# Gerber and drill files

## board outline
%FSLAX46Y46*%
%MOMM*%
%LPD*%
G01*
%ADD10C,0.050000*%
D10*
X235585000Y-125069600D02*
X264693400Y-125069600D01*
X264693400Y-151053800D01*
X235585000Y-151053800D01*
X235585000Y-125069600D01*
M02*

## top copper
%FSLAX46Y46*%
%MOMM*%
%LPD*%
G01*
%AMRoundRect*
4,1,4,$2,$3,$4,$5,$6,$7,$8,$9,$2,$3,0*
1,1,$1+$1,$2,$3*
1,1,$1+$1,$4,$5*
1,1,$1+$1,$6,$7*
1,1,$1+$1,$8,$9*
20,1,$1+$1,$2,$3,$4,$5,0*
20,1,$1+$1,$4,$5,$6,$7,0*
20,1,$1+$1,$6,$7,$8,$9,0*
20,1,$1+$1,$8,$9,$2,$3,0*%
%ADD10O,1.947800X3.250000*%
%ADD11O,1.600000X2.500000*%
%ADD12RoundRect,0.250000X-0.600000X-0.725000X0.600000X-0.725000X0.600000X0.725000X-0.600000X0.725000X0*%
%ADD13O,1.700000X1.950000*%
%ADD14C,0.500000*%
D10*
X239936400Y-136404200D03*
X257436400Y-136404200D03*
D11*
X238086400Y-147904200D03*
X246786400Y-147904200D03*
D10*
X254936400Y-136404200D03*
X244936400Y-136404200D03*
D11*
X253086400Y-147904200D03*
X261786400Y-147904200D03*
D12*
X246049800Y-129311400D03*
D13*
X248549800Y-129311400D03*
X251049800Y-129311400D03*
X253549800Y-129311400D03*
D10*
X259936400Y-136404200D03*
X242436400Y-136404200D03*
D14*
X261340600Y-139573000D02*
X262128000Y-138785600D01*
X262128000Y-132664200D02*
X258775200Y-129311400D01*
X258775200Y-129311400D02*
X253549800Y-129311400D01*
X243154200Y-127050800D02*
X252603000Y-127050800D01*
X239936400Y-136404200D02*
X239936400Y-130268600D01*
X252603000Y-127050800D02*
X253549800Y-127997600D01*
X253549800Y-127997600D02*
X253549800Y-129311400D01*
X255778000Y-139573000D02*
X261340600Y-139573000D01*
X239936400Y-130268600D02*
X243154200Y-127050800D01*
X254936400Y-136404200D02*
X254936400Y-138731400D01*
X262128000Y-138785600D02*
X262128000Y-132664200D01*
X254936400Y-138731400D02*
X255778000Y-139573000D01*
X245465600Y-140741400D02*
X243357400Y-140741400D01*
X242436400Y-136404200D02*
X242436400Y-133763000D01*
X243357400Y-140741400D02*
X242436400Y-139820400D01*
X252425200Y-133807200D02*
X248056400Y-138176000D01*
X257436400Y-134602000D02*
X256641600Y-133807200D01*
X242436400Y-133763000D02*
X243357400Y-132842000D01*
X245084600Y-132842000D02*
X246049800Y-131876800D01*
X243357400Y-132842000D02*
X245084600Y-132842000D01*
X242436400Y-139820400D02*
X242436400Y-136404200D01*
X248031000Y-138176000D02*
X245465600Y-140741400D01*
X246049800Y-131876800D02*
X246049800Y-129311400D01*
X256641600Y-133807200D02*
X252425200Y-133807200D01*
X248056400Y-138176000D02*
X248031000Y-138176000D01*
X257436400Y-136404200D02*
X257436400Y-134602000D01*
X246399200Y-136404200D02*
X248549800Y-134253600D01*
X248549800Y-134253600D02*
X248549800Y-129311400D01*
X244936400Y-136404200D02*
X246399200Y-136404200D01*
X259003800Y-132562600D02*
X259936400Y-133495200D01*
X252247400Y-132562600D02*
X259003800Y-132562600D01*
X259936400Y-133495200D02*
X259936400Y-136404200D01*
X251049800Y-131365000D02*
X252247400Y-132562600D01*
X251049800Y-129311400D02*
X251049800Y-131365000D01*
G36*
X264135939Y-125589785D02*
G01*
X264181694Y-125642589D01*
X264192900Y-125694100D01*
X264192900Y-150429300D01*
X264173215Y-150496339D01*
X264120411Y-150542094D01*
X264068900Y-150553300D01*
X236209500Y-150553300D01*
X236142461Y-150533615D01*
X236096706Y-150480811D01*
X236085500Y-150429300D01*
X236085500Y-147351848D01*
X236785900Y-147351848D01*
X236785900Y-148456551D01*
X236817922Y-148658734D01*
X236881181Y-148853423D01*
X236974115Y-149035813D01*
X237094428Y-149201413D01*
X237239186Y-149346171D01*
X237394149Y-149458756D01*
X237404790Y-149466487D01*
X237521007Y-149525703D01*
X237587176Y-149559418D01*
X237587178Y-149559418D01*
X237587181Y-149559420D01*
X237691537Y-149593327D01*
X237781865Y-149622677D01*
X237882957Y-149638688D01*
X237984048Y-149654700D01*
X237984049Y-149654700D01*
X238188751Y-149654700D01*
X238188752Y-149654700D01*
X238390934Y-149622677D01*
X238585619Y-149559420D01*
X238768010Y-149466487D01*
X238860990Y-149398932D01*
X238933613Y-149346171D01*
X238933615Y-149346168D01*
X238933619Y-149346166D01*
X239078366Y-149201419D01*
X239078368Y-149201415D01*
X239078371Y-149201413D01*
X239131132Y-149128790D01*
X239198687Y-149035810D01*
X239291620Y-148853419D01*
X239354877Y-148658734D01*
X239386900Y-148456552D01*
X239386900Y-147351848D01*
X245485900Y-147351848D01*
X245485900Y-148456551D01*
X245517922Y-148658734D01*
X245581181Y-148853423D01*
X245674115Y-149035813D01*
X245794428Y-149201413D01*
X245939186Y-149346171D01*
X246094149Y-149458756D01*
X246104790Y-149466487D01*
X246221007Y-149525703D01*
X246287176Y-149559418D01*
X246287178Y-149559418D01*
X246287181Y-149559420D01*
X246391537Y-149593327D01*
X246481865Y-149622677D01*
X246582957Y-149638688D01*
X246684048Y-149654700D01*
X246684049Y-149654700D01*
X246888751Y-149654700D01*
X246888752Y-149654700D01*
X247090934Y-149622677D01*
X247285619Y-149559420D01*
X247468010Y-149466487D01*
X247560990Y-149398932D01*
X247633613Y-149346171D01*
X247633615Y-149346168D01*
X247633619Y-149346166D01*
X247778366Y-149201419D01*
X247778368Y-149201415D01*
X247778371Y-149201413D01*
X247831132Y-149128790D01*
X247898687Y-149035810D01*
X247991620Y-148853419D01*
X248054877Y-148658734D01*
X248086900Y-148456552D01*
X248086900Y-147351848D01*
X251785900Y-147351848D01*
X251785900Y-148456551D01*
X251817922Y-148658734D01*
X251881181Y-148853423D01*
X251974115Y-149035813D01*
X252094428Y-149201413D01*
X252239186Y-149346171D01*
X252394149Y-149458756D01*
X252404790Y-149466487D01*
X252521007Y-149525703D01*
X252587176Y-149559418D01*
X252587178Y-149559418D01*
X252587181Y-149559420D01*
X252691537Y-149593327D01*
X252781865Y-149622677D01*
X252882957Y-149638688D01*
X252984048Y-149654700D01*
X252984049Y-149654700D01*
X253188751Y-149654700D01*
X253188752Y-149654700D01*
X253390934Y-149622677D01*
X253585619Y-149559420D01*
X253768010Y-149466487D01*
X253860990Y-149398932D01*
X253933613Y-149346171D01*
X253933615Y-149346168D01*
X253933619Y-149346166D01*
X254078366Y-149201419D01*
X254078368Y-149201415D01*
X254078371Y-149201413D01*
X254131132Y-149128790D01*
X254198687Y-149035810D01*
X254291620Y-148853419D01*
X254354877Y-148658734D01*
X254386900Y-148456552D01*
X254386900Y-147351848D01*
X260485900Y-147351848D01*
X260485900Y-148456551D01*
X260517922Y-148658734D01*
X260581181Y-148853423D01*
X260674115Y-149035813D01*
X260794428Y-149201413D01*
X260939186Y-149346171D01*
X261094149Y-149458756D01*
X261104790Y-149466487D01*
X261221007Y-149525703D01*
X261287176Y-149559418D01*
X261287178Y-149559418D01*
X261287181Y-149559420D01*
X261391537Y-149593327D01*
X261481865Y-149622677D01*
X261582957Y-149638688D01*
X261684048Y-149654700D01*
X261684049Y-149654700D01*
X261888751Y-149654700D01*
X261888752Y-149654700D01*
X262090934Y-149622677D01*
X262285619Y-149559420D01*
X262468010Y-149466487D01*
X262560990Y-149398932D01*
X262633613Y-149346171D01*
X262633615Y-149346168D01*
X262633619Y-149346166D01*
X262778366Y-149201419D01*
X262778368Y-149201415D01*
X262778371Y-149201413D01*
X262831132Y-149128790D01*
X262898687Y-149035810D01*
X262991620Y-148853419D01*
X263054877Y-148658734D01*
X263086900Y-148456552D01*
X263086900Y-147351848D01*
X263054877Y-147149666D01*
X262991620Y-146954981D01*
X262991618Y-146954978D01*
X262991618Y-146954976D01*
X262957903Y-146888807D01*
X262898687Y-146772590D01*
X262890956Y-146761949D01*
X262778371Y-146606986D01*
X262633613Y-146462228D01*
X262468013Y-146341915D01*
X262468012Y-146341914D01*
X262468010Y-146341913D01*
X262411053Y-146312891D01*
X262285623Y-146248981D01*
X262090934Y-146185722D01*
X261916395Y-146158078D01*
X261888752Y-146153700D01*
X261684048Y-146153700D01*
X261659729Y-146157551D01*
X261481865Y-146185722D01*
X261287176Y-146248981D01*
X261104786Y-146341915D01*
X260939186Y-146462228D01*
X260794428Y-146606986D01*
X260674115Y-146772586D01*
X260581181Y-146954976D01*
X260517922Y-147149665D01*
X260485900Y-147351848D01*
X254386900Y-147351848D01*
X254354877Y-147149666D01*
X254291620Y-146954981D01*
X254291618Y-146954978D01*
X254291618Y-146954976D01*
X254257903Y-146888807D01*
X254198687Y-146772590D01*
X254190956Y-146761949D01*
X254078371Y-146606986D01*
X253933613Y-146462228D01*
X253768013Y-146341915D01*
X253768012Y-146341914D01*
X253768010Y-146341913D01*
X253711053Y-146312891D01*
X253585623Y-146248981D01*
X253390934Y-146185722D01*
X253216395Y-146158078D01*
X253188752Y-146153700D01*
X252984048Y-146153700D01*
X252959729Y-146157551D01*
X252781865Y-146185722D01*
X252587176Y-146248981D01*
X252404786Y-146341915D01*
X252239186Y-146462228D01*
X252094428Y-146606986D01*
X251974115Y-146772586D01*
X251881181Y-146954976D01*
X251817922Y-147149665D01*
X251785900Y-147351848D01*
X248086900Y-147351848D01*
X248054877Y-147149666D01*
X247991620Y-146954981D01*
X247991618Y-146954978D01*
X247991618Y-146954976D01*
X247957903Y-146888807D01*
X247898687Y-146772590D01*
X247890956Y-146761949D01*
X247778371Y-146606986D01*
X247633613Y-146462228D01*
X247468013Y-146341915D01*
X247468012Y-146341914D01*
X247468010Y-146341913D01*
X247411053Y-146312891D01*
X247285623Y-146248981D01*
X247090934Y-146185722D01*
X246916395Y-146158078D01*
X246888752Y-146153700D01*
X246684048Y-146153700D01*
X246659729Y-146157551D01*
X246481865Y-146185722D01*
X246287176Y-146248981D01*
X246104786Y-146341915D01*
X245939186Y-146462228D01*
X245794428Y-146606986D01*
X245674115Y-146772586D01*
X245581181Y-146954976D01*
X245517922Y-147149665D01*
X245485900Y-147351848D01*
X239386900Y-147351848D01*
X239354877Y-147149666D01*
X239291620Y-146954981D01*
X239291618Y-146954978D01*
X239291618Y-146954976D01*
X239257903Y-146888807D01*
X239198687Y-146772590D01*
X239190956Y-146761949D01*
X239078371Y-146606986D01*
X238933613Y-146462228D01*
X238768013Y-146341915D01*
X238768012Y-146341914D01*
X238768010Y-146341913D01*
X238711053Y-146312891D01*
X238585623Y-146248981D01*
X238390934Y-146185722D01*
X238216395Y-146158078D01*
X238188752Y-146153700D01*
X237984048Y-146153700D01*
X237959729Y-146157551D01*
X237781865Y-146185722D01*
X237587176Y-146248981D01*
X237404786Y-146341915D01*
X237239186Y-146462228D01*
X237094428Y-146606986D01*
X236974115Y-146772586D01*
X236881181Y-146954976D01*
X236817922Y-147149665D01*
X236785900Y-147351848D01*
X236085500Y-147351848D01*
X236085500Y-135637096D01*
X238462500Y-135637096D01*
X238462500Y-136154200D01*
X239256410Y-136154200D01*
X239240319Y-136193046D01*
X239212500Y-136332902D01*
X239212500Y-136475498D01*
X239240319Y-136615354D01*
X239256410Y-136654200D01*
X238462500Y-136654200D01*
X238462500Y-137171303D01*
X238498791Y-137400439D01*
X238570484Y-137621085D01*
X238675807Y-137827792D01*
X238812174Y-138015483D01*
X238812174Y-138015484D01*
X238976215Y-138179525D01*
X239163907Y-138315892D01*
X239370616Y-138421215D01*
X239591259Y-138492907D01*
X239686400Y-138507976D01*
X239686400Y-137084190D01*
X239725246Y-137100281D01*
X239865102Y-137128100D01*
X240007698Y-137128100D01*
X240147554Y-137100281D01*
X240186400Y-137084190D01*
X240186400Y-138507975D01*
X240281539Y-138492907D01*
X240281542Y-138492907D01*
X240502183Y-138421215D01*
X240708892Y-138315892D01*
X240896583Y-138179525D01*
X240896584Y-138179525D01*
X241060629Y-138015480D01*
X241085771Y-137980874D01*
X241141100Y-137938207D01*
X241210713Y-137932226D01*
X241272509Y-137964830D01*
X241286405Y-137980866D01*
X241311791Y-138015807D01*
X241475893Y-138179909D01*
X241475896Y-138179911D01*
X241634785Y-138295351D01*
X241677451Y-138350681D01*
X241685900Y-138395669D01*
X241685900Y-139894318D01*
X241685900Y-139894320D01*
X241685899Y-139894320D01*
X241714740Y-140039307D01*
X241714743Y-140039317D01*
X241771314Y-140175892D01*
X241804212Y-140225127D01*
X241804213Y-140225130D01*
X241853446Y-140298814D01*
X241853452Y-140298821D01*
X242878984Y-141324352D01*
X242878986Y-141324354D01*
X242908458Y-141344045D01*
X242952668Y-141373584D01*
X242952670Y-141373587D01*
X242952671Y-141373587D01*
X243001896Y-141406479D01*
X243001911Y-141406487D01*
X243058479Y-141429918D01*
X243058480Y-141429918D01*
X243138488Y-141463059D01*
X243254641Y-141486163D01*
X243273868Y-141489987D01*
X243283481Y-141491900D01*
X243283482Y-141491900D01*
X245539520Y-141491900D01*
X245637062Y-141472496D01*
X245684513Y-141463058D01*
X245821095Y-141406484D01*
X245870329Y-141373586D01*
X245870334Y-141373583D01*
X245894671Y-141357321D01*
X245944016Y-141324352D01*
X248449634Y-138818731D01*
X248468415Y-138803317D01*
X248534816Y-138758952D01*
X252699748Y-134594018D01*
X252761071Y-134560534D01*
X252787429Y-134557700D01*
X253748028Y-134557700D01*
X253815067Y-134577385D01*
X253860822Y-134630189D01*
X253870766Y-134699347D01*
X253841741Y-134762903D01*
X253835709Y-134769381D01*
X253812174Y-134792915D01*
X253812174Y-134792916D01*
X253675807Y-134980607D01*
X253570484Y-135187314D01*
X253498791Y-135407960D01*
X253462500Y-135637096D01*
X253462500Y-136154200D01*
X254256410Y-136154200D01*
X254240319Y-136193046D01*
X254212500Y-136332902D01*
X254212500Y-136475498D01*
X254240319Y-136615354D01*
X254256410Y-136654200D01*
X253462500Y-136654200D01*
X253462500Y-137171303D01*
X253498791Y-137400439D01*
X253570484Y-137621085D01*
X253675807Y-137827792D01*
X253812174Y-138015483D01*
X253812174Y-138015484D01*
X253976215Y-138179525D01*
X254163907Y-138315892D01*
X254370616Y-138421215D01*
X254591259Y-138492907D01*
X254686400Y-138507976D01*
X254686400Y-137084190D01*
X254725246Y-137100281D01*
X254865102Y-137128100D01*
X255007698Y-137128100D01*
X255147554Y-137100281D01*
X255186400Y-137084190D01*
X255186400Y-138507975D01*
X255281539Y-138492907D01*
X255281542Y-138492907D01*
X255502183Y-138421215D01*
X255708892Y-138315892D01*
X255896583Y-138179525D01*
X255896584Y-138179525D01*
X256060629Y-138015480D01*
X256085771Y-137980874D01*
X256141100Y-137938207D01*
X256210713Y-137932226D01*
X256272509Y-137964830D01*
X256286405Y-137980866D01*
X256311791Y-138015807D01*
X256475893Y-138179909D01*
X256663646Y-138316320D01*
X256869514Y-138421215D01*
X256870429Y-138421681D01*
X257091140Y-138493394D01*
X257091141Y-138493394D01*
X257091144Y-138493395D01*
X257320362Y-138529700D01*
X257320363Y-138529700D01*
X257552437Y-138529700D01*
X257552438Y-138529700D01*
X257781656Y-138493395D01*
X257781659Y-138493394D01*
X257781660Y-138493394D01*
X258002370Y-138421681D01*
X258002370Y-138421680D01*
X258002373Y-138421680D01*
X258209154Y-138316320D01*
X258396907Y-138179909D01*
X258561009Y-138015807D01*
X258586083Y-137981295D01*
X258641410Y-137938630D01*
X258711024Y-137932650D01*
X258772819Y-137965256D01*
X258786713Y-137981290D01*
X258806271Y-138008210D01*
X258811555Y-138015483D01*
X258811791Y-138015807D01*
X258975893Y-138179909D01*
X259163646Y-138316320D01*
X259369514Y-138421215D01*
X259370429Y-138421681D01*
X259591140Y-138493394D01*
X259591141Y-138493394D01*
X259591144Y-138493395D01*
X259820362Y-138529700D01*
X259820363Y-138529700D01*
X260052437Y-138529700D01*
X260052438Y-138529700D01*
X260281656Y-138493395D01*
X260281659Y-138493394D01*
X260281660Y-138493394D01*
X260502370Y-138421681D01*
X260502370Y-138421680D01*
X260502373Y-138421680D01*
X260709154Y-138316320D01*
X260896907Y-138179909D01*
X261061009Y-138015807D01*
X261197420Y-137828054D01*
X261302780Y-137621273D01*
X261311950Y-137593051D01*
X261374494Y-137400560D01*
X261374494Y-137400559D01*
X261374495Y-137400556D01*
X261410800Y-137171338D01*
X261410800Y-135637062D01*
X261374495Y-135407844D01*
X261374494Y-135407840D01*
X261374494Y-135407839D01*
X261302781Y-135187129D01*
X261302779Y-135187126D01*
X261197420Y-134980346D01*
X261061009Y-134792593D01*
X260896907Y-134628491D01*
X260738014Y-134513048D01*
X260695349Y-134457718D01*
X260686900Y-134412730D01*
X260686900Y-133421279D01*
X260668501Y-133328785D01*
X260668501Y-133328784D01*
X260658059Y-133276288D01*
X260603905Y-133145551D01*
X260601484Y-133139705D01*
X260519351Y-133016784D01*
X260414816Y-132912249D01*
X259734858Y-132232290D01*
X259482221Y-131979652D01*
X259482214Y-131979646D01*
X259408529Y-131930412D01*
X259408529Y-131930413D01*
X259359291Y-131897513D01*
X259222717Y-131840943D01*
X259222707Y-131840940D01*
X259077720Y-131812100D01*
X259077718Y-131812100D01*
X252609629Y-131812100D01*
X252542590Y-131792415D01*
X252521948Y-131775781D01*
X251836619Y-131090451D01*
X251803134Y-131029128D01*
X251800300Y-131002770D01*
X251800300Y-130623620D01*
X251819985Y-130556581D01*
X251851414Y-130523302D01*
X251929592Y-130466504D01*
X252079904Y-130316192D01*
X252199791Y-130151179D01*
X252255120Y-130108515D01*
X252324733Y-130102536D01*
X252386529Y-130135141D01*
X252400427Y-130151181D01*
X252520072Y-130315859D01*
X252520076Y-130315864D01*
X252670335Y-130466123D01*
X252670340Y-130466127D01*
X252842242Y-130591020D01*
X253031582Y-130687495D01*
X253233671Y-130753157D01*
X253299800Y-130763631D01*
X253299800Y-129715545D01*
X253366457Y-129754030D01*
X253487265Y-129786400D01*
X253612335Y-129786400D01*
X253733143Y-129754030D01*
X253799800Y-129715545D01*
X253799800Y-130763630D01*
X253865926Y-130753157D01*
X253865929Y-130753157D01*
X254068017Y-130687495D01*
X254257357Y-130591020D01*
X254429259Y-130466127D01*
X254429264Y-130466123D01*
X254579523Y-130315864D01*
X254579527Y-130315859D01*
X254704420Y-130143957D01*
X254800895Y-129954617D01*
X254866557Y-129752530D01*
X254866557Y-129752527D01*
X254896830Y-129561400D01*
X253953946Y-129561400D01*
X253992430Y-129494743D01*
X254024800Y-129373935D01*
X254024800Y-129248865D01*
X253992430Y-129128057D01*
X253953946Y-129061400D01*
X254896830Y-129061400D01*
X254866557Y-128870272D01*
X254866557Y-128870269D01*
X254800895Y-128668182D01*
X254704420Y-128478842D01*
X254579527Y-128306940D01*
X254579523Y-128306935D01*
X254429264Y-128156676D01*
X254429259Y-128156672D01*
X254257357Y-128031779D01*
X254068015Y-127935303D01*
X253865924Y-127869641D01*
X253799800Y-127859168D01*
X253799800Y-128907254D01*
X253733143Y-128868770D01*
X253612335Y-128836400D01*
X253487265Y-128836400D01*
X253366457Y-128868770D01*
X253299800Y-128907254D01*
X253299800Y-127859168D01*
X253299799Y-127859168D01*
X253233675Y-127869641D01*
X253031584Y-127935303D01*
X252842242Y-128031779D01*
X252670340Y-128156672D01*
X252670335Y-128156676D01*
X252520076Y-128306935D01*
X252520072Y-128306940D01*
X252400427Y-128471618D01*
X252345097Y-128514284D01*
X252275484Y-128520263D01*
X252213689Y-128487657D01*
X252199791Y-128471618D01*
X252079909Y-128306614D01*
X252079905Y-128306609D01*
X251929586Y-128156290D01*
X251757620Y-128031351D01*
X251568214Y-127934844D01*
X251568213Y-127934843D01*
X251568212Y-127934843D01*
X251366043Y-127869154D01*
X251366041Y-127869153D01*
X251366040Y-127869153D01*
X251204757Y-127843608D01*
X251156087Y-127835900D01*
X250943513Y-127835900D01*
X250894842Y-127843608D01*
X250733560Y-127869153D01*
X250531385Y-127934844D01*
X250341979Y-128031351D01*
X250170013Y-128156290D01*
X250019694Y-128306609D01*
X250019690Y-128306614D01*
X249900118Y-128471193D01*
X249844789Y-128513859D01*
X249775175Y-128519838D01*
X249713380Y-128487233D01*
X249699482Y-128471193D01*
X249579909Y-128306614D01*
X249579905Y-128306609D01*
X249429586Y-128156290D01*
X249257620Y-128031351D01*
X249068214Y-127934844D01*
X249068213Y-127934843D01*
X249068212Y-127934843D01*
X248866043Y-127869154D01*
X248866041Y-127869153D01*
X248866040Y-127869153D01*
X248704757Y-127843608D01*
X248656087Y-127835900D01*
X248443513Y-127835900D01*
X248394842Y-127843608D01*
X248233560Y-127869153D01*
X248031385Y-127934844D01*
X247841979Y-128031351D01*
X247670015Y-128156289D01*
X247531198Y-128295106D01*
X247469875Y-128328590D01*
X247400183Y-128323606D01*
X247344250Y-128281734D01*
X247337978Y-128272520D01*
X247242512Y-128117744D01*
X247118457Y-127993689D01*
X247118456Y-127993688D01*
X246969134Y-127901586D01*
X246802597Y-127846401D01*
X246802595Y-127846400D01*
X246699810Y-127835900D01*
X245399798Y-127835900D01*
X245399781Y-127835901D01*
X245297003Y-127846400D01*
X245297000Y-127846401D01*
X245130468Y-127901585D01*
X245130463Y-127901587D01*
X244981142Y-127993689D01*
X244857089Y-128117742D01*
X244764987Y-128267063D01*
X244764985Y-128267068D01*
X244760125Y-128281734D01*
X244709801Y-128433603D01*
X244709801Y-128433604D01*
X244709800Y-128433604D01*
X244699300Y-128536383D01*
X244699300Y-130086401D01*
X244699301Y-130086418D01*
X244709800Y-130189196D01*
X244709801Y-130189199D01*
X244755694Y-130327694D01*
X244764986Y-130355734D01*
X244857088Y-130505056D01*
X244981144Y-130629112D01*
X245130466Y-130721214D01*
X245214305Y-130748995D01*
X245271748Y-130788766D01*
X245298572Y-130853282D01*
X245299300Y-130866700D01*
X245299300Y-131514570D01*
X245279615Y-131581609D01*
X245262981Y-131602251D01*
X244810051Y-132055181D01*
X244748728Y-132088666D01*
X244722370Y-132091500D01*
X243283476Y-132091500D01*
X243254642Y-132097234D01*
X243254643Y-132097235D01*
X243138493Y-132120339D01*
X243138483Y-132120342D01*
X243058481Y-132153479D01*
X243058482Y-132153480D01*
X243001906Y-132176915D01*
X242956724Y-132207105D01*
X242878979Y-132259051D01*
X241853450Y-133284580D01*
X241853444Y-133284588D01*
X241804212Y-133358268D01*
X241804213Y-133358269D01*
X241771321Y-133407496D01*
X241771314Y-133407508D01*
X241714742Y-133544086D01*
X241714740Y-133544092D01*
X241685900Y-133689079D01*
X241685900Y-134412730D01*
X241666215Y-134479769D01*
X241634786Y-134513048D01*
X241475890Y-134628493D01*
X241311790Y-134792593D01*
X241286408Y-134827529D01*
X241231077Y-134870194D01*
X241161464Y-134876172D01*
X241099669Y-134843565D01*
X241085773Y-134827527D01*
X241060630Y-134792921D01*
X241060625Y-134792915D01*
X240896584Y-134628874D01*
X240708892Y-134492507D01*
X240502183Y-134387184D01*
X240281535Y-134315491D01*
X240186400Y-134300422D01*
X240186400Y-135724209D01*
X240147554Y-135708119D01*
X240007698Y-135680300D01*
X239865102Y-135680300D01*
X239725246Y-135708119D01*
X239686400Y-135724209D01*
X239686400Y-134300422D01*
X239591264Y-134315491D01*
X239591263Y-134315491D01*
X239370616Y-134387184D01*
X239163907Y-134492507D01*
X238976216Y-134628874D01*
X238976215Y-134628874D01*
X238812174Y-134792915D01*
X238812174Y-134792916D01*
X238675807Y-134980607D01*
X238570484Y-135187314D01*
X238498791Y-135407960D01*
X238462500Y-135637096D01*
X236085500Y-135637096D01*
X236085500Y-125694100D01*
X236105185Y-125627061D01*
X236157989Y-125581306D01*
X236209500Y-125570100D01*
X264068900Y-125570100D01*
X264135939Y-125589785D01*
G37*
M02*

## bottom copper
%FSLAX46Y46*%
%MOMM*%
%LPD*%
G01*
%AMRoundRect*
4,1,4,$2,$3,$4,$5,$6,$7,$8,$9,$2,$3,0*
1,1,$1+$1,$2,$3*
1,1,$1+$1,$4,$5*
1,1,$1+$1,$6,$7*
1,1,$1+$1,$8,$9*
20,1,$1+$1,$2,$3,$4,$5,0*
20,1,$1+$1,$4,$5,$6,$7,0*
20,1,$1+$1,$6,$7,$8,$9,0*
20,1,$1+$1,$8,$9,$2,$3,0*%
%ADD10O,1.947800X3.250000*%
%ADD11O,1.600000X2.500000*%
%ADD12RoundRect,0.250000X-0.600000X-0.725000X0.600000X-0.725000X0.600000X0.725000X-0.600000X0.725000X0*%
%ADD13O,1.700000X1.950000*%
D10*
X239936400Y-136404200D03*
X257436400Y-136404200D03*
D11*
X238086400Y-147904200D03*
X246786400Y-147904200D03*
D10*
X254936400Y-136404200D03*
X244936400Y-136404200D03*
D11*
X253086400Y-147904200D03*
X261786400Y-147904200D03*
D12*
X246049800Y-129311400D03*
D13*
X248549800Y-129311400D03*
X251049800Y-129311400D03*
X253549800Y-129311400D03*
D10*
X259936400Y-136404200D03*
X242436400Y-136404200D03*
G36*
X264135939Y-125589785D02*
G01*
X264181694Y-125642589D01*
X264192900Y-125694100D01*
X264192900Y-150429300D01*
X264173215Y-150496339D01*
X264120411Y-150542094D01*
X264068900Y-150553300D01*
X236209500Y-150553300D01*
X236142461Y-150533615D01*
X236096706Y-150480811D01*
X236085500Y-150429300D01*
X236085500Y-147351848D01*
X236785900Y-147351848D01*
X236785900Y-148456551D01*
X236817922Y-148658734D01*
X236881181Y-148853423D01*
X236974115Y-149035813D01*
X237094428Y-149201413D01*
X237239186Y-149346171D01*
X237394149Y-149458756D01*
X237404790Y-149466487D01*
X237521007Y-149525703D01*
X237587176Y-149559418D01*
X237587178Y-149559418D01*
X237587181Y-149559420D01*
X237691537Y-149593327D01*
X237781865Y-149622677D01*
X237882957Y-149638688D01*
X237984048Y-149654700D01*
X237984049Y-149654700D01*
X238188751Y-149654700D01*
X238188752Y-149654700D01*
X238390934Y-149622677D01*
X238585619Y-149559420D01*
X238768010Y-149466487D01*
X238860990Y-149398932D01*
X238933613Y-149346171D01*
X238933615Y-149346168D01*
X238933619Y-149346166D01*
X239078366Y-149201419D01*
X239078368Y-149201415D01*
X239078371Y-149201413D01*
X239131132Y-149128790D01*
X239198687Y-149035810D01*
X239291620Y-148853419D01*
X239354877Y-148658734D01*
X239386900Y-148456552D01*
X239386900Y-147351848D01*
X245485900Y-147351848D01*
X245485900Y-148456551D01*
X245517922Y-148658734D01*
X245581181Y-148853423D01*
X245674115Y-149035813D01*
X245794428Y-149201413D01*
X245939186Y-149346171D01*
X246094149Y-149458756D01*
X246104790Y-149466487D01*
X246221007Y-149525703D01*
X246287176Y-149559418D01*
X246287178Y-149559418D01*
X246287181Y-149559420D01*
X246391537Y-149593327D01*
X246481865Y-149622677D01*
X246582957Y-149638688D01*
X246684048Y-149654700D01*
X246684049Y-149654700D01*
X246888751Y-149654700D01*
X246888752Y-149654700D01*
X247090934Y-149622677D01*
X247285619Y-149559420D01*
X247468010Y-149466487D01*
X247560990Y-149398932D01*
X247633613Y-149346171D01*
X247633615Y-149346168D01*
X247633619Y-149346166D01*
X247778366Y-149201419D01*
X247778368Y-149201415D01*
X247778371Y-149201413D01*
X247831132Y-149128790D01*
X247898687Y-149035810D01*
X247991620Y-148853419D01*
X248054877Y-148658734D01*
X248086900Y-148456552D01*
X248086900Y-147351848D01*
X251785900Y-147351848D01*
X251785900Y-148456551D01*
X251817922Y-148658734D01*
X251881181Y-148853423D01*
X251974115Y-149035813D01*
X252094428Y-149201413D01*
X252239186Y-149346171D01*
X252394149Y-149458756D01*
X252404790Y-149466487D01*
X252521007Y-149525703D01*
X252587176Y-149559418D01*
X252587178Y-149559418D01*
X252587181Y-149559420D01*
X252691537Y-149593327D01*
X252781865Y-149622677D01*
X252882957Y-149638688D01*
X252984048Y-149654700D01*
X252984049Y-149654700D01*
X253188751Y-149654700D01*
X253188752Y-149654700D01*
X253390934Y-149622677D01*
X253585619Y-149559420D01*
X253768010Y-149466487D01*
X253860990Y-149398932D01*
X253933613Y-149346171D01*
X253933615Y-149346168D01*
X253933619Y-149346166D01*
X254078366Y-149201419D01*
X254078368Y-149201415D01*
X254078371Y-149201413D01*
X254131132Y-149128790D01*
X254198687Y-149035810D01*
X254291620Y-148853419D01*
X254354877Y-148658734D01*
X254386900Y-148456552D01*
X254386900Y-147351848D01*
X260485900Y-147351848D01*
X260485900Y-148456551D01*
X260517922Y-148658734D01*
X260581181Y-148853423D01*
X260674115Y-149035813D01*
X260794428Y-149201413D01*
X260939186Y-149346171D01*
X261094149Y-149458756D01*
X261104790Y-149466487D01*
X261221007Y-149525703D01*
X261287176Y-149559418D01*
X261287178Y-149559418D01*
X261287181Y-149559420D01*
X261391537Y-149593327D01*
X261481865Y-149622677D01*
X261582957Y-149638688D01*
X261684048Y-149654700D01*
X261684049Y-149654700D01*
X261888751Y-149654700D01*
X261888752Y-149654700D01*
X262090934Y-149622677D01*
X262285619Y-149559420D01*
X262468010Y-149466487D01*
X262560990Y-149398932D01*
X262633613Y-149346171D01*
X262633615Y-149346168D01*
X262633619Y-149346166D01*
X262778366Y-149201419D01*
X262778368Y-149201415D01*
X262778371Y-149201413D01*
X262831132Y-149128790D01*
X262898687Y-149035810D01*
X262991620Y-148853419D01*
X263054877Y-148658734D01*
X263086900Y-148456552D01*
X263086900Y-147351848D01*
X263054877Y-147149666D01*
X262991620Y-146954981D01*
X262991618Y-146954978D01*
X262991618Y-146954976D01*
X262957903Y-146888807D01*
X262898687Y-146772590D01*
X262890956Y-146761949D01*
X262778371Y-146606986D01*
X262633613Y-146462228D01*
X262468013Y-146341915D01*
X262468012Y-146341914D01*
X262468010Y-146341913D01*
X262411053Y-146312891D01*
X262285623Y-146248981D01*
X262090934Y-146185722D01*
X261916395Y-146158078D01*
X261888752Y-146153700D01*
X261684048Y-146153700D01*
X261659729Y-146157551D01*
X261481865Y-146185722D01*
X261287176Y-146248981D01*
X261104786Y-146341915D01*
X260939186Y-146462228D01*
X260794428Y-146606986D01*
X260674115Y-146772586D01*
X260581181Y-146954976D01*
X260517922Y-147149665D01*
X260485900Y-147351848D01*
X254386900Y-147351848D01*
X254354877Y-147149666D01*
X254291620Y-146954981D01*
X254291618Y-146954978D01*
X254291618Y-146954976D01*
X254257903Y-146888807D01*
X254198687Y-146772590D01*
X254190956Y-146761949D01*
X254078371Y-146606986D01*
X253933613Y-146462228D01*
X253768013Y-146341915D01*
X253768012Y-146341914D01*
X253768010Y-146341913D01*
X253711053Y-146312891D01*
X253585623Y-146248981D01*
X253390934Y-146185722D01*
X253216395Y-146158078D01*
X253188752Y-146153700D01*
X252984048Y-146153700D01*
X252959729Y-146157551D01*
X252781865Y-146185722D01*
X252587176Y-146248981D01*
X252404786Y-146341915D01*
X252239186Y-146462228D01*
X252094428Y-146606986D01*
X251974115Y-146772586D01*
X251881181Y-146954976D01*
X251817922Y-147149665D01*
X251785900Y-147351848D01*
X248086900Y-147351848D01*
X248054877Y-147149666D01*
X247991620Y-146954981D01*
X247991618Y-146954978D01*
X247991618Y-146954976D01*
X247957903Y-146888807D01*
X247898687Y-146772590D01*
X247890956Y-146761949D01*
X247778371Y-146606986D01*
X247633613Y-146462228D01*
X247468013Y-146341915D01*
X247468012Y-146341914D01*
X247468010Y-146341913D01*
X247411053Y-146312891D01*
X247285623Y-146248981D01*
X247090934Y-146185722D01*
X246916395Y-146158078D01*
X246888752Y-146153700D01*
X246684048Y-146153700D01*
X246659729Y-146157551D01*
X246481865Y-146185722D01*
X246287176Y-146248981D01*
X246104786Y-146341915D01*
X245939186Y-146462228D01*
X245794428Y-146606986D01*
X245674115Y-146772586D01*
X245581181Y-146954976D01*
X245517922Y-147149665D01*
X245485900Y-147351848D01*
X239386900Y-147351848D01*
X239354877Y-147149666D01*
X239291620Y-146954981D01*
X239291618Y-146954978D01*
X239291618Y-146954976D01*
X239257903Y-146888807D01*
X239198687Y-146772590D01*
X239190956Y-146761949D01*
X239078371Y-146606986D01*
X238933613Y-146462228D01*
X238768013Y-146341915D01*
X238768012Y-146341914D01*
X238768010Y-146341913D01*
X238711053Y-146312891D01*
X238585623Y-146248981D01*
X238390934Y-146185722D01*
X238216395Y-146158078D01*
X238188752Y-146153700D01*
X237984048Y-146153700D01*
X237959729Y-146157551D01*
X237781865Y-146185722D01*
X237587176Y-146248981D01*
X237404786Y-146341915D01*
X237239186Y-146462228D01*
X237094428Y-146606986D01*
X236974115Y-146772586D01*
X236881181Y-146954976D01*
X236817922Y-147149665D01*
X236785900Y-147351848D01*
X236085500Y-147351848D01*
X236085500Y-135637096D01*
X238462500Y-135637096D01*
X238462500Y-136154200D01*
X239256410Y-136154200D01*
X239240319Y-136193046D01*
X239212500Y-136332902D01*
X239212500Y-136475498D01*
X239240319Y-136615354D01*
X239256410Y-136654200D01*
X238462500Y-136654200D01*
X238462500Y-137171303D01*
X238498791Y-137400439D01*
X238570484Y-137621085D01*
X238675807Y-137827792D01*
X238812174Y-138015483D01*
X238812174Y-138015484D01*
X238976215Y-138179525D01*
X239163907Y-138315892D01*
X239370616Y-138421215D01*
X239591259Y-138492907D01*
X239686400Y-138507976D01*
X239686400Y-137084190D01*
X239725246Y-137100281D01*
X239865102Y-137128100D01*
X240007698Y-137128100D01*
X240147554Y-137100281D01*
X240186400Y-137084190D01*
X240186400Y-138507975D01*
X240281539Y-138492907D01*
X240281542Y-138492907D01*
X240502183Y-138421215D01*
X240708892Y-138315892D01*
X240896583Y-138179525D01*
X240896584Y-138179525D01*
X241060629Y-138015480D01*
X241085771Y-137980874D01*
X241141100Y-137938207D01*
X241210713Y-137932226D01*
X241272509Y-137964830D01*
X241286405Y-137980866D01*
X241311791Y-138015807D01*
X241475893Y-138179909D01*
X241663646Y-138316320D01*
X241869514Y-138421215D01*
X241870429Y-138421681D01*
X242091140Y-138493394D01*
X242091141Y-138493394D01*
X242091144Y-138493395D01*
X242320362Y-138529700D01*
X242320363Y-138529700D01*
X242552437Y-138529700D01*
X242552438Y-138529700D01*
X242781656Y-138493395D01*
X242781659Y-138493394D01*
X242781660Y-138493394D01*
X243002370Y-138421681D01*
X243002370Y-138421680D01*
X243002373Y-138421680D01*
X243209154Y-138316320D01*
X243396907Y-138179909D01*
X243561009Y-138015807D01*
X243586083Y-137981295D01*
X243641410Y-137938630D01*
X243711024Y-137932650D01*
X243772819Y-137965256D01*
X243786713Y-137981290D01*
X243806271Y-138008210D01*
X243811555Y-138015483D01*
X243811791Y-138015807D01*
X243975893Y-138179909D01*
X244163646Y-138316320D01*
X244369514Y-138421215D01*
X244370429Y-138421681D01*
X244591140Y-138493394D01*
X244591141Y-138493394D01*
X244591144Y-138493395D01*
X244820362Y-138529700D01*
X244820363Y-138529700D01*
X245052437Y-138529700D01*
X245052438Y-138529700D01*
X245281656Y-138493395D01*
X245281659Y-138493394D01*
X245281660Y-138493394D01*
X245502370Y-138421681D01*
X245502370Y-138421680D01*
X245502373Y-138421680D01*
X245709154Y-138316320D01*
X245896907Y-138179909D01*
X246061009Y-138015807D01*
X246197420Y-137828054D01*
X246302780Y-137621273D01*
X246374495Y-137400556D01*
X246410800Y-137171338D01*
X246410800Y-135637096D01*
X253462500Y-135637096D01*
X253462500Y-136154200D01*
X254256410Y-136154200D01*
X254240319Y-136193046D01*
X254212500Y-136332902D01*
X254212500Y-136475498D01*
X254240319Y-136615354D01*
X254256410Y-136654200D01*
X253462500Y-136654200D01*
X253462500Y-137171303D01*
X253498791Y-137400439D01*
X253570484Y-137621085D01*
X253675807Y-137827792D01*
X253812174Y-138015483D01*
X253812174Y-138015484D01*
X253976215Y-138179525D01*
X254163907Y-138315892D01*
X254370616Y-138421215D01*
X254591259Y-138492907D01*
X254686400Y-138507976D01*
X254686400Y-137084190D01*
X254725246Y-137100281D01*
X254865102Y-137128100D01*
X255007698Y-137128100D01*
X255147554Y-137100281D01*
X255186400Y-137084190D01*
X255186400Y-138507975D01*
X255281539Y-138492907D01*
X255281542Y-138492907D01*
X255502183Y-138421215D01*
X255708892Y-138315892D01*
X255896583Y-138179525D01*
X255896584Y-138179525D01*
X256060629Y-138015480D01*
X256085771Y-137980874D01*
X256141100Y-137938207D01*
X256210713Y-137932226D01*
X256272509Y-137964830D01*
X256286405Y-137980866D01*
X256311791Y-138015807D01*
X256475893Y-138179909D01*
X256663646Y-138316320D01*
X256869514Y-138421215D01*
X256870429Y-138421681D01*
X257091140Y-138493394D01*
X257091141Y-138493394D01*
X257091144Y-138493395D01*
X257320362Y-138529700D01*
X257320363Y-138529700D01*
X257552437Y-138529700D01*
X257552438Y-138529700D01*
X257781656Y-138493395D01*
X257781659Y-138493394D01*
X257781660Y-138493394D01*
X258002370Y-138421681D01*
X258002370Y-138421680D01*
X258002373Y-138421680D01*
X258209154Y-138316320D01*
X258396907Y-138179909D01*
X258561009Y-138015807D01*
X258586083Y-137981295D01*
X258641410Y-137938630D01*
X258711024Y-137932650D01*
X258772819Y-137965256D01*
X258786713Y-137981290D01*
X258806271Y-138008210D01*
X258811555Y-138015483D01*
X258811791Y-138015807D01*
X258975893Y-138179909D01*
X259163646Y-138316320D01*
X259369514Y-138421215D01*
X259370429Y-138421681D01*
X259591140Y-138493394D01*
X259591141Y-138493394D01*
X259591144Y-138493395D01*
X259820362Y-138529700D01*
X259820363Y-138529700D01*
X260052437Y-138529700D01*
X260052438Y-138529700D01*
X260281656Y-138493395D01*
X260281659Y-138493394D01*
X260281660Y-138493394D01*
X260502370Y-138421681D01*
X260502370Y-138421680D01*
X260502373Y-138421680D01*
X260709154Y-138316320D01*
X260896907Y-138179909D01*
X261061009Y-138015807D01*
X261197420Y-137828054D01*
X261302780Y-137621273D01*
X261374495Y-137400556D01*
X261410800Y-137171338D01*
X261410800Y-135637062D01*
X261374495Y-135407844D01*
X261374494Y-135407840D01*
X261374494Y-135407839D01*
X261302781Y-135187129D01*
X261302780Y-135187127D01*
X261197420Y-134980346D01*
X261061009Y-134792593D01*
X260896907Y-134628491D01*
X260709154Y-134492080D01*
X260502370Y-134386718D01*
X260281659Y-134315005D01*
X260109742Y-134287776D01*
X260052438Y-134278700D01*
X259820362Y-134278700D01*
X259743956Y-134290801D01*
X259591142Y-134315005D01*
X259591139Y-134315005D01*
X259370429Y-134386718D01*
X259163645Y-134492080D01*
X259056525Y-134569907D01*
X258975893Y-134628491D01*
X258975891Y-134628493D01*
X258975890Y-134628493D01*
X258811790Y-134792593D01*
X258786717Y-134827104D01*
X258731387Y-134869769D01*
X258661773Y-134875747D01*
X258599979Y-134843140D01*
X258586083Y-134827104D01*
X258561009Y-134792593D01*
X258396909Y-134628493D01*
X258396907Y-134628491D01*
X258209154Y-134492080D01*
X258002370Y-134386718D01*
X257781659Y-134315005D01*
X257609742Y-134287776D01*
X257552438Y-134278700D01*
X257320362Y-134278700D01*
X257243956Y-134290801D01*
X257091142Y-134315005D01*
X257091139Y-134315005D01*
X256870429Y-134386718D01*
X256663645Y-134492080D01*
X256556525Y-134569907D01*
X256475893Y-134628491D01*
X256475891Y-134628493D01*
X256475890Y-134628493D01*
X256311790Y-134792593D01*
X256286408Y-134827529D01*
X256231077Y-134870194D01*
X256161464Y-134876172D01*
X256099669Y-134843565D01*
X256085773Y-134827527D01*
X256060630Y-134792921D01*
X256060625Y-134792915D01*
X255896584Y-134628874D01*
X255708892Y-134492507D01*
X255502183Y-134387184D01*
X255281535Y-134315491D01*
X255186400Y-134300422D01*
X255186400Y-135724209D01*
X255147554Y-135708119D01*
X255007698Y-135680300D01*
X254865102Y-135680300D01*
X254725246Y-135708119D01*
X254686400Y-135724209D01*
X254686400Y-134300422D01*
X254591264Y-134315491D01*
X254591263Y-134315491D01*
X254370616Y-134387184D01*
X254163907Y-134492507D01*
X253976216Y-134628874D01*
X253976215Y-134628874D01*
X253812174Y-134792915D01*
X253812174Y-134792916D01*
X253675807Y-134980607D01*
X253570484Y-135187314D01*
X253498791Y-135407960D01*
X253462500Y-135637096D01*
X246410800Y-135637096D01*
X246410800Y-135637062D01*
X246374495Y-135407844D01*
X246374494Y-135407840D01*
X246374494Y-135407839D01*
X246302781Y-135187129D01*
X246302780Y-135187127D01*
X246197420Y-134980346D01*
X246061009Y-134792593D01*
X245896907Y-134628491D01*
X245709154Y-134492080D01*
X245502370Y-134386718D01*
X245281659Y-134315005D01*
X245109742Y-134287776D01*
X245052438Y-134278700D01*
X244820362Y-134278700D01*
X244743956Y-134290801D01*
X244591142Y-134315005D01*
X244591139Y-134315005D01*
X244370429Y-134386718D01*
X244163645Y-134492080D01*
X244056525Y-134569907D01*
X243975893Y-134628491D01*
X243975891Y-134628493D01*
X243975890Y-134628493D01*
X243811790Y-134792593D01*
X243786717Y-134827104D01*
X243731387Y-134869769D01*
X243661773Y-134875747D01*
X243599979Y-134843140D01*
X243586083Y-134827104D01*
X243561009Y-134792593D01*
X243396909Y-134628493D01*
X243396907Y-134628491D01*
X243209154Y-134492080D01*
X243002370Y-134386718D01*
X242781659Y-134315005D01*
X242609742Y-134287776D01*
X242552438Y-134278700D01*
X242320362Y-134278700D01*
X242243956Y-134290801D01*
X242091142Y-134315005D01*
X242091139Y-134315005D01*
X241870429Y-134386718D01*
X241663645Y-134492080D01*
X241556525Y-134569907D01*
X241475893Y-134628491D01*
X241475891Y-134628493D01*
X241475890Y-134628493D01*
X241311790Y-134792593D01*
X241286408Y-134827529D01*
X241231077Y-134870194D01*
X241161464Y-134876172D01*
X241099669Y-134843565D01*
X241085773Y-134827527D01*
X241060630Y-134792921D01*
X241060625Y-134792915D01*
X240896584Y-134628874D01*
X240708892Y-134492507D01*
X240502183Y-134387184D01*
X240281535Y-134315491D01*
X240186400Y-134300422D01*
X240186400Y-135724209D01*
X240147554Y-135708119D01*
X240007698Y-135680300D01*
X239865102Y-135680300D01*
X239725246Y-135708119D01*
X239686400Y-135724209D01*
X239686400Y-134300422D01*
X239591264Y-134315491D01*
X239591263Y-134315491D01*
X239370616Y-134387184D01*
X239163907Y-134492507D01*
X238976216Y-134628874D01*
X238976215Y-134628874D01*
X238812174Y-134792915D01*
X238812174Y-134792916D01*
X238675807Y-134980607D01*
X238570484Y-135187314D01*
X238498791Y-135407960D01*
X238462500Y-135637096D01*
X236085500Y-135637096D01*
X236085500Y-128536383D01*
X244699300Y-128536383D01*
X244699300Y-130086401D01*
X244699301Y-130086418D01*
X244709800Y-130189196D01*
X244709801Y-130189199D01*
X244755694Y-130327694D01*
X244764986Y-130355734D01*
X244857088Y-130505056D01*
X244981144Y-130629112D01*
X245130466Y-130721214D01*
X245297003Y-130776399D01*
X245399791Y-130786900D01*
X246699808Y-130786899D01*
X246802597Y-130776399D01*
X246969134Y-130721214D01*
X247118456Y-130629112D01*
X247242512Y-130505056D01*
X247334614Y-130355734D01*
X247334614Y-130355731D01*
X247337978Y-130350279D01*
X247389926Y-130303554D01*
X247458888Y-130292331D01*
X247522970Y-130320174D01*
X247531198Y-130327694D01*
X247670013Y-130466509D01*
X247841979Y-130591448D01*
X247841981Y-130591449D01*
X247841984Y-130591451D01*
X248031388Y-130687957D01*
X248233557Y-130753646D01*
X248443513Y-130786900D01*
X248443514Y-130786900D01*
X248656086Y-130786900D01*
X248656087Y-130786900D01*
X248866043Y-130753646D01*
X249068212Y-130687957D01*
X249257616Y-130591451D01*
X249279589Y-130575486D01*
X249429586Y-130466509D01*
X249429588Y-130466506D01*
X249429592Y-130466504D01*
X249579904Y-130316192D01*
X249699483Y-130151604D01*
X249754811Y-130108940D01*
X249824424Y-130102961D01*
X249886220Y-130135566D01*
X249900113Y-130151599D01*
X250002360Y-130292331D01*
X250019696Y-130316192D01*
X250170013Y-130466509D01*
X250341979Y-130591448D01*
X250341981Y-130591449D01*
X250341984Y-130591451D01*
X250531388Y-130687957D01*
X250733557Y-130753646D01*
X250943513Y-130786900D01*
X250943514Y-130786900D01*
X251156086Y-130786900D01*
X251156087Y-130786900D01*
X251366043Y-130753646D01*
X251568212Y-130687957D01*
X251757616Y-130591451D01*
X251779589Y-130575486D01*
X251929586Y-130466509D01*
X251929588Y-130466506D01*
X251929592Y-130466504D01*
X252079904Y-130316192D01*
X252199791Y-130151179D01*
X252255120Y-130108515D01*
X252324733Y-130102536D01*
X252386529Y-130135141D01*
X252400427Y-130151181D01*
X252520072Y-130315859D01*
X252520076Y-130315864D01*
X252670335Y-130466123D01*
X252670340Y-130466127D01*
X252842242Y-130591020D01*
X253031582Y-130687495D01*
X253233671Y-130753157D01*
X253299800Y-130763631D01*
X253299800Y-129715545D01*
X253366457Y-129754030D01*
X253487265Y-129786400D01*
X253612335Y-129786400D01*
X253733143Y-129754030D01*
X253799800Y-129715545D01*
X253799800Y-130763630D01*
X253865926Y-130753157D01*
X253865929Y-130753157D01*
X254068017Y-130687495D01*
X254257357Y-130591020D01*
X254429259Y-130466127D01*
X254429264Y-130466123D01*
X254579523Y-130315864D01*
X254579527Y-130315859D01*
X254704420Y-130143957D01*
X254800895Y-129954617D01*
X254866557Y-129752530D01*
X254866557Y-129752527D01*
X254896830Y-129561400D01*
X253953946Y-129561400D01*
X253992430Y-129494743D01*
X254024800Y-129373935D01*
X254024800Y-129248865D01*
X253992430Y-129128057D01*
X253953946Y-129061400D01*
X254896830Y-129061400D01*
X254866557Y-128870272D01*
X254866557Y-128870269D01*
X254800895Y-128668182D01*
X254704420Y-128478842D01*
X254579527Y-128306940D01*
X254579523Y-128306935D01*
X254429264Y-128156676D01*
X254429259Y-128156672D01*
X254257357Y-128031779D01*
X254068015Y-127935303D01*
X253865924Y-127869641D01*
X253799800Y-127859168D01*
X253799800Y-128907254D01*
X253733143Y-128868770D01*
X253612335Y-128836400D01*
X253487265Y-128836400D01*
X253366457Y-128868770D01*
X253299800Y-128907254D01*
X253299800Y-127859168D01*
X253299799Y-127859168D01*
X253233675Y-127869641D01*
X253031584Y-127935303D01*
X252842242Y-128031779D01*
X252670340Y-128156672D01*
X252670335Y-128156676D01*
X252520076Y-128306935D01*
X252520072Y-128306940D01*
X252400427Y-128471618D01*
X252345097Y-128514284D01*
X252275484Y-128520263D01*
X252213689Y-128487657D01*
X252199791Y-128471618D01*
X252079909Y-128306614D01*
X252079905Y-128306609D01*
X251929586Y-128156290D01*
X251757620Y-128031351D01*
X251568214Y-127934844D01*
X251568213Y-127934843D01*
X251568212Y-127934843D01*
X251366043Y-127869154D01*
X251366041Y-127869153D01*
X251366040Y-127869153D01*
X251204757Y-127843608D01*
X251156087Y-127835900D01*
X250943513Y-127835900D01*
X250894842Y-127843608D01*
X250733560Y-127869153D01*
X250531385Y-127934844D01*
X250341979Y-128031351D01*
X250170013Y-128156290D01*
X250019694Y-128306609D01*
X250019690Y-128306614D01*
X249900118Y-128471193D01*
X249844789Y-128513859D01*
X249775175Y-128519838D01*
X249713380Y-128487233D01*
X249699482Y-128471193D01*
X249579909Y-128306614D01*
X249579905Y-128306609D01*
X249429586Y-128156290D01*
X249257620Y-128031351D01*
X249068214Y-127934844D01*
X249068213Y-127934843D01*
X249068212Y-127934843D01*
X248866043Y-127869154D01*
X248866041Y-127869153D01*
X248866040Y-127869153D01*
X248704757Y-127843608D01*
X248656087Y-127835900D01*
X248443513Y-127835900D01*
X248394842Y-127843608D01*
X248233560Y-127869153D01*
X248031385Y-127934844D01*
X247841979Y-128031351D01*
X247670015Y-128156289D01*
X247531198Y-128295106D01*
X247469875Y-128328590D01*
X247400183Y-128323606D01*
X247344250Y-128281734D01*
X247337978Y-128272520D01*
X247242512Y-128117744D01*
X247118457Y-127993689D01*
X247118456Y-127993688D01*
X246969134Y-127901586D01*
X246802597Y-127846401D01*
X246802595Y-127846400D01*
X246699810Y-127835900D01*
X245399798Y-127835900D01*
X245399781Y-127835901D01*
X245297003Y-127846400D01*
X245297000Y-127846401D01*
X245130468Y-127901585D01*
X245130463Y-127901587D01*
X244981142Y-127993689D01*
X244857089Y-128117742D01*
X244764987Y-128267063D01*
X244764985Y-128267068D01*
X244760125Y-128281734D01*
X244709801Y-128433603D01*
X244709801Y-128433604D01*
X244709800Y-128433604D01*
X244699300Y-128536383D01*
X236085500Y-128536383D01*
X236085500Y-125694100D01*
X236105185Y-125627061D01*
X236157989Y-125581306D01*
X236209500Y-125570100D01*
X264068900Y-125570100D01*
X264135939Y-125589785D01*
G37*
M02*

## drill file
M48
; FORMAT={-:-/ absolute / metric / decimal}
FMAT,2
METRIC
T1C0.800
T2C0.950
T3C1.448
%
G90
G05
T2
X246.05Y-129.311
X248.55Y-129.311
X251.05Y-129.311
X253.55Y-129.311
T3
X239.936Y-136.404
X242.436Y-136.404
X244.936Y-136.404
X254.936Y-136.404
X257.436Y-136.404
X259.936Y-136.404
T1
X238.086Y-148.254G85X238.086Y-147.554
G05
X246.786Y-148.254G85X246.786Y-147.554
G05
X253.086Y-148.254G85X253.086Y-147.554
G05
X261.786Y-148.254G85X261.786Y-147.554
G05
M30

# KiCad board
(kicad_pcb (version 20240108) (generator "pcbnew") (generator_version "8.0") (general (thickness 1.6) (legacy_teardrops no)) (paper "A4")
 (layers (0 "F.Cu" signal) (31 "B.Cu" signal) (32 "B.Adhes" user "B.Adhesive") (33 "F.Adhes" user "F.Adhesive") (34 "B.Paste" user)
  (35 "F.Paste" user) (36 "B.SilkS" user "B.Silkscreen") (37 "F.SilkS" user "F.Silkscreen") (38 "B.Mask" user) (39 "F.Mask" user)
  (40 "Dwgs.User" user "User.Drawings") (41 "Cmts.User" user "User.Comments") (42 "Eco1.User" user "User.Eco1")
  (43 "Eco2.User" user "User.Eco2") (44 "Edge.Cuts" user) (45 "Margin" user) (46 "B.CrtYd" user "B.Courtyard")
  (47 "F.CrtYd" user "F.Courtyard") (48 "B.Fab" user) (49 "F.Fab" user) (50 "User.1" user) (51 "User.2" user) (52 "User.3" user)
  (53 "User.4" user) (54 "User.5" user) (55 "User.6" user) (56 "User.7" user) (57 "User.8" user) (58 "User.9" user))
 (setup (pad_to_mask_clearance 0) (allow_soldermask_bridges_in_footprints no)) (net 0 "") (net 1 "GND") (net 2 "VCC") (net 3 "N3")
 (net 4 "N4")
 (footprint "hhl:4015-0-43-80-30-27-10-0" (layer "F.Cu") (at 239.9364 136.4042)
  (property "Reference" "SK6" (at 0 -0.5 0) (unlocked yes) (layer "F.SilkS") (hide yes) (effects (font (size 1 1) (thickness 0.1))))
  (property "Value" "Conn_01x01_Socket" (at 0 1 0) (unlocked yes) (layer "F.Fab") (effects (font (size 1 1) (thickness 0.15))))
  (pad "1" thru_hole oval (at 0 0) (size 1.9478 3.25) (drill 1.4478) (layers "*.Cu" "*.Mask") (remove_unused_layers no) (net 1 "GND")))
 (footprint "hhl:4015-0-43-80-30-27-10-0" (layer "F.Cu") (at 257.4364 136.4042)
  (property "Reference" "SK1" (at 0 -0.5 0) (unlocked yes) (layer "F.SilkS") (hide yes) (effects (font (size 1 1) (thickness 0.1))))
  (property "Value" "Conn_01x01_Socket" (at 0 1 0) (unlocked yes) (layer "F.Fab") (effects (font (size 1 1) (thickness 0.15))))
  (pad "1" thru_hole oval (at 0 0) (size 1.9478 3.25) (drill 1.4478) (layers "*.Cu" "*.Mask") (remove_unused_layers no) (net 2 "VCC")))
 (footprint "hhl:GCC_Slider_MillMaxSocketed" (layer "F.Cu") (at 242.4364 136.4042)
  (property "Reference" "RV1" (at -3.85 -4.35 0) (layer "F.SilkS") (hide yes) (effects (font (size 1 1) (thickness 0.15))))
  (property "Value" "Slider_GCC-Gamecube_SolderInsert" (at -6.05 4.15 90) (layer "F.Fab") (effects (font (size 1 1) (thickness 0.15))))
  (pad "MP" thru_hole oval (at -4.35 11.5 180) (size 1.6 2.5) (drill oval 0.8 1.5) (layers "*.Cu" "*.Mask") (remove_unused_layers no))
  (pad "MP" thru_hole oval (at 4.35 11.5 180) (size 1.6 2.5) (drill oval 0.8 1.5) (layers "*.Cu" "*.Mask") (remove_unused_layers no)))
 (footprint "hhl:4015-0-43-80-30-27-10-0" (layer "F.Cu") (at 254.9364 136.4042)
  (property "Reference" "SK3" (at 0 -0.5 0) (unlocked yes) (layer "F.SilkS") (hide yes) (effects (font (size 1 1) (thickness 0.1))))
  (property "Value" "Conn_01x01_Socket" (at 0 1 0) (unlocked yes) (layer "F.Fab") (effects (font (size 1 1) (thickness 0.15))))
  (pad "1" thru_hole oval (at 0 0) (size 1.9478 3.25) (drill 1.4478) (layers "*.Cu" "*.Mask") (remove_unused_layers no) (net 1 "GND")))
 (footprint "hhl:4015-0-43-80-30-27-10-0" (layer "F.Cu") (at 244.9364 136.4042)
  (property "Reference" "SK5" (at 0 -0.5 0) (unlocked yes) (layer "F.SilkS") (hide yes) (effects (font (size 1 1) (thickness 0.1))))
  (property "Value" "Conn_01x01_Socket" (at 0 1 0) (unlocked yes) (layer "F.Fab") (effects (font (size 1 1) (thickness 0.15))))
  (pad "1" thru_hole oval (at 0 0) (size 1.9478 3.25) (drill 1.4478) (layers "*.Cu" "*.Mask") (remove_unused_layers no) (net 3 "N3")))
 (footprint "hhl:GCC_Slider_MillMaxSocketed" (layer "F.Cu") (at 257.4364 136.4042)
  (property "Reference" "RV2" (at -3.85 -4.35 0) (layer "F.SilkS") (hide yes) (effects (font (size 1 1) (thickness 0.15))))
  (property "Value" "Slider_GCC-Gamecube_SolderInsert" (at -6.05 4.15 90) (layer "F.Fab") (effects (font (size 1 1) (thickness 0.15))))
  (pad "MP" thru_hole oval (at -4.35 11.5 180) (size 1.6 2.5) (drill oval 0.8 1.5) (layers "*.Cu" "*.Mask") (remove_unused_layers no))
  (pad "MP" thru_hole oval (at 4.35 11.5 180) (size 1.6 2.5) (drill oval 0.8 1.5) (layers "*.Cu" "*.Mask") (remove_unused_layers no)))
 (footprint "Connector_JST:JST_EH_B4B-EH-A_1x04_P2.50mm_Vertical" (layer "F.Cu") (at 246.0498 129.3114)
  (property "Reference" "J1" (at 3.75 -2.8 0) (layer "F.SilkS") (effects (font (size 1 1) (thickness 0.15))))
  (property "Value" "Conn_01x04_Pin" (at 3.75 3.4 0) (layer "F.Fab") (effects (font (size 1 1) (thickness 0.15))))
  (pad "1" thru_hole roundrect (at 0 0) (size 1.7 1.95) (drill 0.95) (layers "*.Cu" "*.Mask") (remove_unused_layers no)
   (roundrect_rratio 0.147059) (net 2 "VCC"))
  (pad "2" thru_hole oval (at 2.5 0) (size 1.7 1.95) (drill 0.95) (layers "*.Cu" "*.Mask") (remove_unused_layers no) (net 3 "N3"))
  (pad "3" thru_hole oval (at 5 0) (size 1.7 1.95) (drill 0.95) (layers "*.Cu" "*.Mask") (remove_unused_layers no) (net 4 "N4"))
  (pad "4" thru_hole oval (at 7.5 0) (size 1.7 1.95) (drill 0.95) (layers "*.Cu" "*.Mask") (remove_unused_layers no) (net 1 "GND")))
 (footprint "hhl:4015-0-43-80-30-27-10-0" (layer "F.Cu") (at 259.9364 136.4042)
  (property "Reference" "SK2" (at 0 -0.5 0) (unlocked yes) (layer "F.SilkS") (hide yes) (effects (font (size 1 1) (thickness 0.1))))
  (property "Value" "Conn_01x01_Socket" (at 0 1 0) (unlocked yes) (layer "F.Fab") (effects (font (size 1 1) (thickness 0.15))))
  (pad "1" thru_hole oval (at 0 0) (size 1.9478 3.25) (drill 1.4478) (layers "*.Cu" "*.Mask") (remove_unused_layers no) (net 4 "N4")))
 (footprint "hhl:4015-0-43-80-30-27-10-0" (layer "F.Cu") (at 242.4364 136.4042)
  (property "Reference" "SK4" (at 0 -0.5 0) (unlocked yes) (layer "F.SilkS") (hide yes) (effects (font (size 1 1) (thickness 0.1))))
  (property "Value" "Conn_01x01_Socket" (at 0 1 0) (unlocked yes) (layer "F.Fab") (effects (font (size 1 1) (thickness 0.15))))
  (pad "1" thru_hole oval (at 0 0) (size 1.9478 3.25) (drill 1.4478) (layers "*.Cu" "*.Mask") (remove_unused_layers no) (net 2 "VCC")))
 (gr_rect (start 235.585 125.0696) (end 264.6934 151.0538) (stroke (width 0.05) (type default)) (fill none) (layer "Edge.Cuts"))
 (segment (start 261.3406 139.573) (end 262.128 138.7856) (width 0.5) (layer "F.Cu") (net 1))
 (segment (start 262.128 132.6642) (end 258.7752 129.3114) (width 0.5) (layer "F.Cu") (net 1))
 (segment (start 258.7752 129.3114) (end 253.5498 129.3114) (width 0.5) (layer "F.Cu") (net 1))
 (segment (start 243.1542 127.0508) (end 252.603 127.0508) (width 0.5) (layer "F.Cu") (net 1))
 (segment (start 239.9364 136.4042) (end 239.9364 130.2686) (width 0.5) (layer "F.Cu") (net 1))
 (segment (start 252.603 127.0508) (end 253.5498 127.9976) (width 0.5) (layer "F.Cu") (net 1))
 (segment (start 253.5498 127.9976) (end 253.5498 129.3114) (width 0.5) (layer "F.Cu") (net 1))
 (segment (start 255.778 139.573) (end 261.3406 139.573) (width 0.5) (layer "F.Cu") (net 1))
 (segment (start 239.9364 130.2686) (end 243.1542 127.0508) (width 0.5) (layer "F.Cu") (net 1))
 (segment (start 254.9364 136.4042) (end 254.9364 138.7314) (width 0.5) (layer "F.Cu") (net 1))
 (segment (start 262.128 138.7856) (end 262.128 132.6642) (width 0.5) (layer "F.Cu") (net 1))
 (segment (start 254.9364 138.7314) (end 255.778 139.573) (width 0.5) (layer "F.Cu") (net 1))
 (segment (start 245.4656 140.7414) (end 243.3574 140.7414) (width 0.5) (layer "F.Cu") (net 2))
 (segment (start 242.4364 136.4042) (end 242.4364 133.763) (width 0.5) (layer "F.Cu") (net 2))
 (segment (start 243.3574 140.7414) (end 242.4364 139.8204) (width 0.5) (layer "F.Cu") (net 2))
 (segment (start 252.4252 133.8072) (end 248.0564 138.176) (width 0.5) (layer "F.Cu") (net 2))
 (segment (start 257.4364 134.602) (end 256.6416 133.8072) (width 0.5) (layer "F.Cu") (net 2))
 (segment (start 242.4364 133.763) (end 243.3574 132.842) (width 0.5) (layer "F.Cu") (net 2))
 (segment (start 245.0846 132.842) (end 246.0498 131.8768) (width 0.5) (layer "F.Cu") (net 2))
 (segment (start 243.3574 132.842) (end 245.0846 132.842) (width 0.5) (layer "F.Cu") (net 2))
 (segment (start 242.4364 139.8204) (end 242.4364 136.4042) (width 0.5) (layer "F.Cu") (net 2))
 (segment (start 248.031 138.176) (end 245.4656 140.7414) (width 0.5) (layer "F.Cu") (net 2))
 (segment (start 246.0498 131.8768) (end 246.0498 129.3114) (width 0.5) (layer "F.Cu") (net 2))
 (segment (start 256.6416 133.8072) (end 252.4252 133.8072) (width 0.5) (layer "F.Cu") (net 2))
 (segment (start 248.0564 138.176) (end 248.031 138.176) (width 0.5) (layer "F.Cu") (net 2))
 (segment (start 257.4364 136.4042) (end 257.4364 134.602) (width 0.5) (layer "F.Cu") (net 2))
 (segment (start 246.3992 136.4042) (end 248.5498 134.2536) (width 0.5) (layer "F.Cu") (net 3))
 (segment (start 248.5498 134.2536) (end 248.5498 129.3114) (width 0.5) (layer "F.Cu") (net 3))
 (segment (start 244.9364 136.4042) (end 246.3992 136.4042) (width 0.5) (layer "F.Cu") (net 3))
 (segment (start 259.0038 132.5626) (end 259.9364 133.4952) (width 0.5) (layer "F.Cu") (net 4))
 (segment (start 252.2474 132.5626) (end 259.0038 132.5626) (width 0.5) (layer "F.Cu") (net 4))
 (segment (start 259.9364 133.4952) (end 259.9364 136.4042) (width 0.5) (layer "F.Cu") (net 4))
 (segment (start 251.0498 131.365) (end 252.2474 132.5626) (width 0.5) (layer "F.Cu") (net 4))
 (segment (start 251.0498 129.3114) (end 251.0498 131.365) (width 0.5) (layer "F.Cu") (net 4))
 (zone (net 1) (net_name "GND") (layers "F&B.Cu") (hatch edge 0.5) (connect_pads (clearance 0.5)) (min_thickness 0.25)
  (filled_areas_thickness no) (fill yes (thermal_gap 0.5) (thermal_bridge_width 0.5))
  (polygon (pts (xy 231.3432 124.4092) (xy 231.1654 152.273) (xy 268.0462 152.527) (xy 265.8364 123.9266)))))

